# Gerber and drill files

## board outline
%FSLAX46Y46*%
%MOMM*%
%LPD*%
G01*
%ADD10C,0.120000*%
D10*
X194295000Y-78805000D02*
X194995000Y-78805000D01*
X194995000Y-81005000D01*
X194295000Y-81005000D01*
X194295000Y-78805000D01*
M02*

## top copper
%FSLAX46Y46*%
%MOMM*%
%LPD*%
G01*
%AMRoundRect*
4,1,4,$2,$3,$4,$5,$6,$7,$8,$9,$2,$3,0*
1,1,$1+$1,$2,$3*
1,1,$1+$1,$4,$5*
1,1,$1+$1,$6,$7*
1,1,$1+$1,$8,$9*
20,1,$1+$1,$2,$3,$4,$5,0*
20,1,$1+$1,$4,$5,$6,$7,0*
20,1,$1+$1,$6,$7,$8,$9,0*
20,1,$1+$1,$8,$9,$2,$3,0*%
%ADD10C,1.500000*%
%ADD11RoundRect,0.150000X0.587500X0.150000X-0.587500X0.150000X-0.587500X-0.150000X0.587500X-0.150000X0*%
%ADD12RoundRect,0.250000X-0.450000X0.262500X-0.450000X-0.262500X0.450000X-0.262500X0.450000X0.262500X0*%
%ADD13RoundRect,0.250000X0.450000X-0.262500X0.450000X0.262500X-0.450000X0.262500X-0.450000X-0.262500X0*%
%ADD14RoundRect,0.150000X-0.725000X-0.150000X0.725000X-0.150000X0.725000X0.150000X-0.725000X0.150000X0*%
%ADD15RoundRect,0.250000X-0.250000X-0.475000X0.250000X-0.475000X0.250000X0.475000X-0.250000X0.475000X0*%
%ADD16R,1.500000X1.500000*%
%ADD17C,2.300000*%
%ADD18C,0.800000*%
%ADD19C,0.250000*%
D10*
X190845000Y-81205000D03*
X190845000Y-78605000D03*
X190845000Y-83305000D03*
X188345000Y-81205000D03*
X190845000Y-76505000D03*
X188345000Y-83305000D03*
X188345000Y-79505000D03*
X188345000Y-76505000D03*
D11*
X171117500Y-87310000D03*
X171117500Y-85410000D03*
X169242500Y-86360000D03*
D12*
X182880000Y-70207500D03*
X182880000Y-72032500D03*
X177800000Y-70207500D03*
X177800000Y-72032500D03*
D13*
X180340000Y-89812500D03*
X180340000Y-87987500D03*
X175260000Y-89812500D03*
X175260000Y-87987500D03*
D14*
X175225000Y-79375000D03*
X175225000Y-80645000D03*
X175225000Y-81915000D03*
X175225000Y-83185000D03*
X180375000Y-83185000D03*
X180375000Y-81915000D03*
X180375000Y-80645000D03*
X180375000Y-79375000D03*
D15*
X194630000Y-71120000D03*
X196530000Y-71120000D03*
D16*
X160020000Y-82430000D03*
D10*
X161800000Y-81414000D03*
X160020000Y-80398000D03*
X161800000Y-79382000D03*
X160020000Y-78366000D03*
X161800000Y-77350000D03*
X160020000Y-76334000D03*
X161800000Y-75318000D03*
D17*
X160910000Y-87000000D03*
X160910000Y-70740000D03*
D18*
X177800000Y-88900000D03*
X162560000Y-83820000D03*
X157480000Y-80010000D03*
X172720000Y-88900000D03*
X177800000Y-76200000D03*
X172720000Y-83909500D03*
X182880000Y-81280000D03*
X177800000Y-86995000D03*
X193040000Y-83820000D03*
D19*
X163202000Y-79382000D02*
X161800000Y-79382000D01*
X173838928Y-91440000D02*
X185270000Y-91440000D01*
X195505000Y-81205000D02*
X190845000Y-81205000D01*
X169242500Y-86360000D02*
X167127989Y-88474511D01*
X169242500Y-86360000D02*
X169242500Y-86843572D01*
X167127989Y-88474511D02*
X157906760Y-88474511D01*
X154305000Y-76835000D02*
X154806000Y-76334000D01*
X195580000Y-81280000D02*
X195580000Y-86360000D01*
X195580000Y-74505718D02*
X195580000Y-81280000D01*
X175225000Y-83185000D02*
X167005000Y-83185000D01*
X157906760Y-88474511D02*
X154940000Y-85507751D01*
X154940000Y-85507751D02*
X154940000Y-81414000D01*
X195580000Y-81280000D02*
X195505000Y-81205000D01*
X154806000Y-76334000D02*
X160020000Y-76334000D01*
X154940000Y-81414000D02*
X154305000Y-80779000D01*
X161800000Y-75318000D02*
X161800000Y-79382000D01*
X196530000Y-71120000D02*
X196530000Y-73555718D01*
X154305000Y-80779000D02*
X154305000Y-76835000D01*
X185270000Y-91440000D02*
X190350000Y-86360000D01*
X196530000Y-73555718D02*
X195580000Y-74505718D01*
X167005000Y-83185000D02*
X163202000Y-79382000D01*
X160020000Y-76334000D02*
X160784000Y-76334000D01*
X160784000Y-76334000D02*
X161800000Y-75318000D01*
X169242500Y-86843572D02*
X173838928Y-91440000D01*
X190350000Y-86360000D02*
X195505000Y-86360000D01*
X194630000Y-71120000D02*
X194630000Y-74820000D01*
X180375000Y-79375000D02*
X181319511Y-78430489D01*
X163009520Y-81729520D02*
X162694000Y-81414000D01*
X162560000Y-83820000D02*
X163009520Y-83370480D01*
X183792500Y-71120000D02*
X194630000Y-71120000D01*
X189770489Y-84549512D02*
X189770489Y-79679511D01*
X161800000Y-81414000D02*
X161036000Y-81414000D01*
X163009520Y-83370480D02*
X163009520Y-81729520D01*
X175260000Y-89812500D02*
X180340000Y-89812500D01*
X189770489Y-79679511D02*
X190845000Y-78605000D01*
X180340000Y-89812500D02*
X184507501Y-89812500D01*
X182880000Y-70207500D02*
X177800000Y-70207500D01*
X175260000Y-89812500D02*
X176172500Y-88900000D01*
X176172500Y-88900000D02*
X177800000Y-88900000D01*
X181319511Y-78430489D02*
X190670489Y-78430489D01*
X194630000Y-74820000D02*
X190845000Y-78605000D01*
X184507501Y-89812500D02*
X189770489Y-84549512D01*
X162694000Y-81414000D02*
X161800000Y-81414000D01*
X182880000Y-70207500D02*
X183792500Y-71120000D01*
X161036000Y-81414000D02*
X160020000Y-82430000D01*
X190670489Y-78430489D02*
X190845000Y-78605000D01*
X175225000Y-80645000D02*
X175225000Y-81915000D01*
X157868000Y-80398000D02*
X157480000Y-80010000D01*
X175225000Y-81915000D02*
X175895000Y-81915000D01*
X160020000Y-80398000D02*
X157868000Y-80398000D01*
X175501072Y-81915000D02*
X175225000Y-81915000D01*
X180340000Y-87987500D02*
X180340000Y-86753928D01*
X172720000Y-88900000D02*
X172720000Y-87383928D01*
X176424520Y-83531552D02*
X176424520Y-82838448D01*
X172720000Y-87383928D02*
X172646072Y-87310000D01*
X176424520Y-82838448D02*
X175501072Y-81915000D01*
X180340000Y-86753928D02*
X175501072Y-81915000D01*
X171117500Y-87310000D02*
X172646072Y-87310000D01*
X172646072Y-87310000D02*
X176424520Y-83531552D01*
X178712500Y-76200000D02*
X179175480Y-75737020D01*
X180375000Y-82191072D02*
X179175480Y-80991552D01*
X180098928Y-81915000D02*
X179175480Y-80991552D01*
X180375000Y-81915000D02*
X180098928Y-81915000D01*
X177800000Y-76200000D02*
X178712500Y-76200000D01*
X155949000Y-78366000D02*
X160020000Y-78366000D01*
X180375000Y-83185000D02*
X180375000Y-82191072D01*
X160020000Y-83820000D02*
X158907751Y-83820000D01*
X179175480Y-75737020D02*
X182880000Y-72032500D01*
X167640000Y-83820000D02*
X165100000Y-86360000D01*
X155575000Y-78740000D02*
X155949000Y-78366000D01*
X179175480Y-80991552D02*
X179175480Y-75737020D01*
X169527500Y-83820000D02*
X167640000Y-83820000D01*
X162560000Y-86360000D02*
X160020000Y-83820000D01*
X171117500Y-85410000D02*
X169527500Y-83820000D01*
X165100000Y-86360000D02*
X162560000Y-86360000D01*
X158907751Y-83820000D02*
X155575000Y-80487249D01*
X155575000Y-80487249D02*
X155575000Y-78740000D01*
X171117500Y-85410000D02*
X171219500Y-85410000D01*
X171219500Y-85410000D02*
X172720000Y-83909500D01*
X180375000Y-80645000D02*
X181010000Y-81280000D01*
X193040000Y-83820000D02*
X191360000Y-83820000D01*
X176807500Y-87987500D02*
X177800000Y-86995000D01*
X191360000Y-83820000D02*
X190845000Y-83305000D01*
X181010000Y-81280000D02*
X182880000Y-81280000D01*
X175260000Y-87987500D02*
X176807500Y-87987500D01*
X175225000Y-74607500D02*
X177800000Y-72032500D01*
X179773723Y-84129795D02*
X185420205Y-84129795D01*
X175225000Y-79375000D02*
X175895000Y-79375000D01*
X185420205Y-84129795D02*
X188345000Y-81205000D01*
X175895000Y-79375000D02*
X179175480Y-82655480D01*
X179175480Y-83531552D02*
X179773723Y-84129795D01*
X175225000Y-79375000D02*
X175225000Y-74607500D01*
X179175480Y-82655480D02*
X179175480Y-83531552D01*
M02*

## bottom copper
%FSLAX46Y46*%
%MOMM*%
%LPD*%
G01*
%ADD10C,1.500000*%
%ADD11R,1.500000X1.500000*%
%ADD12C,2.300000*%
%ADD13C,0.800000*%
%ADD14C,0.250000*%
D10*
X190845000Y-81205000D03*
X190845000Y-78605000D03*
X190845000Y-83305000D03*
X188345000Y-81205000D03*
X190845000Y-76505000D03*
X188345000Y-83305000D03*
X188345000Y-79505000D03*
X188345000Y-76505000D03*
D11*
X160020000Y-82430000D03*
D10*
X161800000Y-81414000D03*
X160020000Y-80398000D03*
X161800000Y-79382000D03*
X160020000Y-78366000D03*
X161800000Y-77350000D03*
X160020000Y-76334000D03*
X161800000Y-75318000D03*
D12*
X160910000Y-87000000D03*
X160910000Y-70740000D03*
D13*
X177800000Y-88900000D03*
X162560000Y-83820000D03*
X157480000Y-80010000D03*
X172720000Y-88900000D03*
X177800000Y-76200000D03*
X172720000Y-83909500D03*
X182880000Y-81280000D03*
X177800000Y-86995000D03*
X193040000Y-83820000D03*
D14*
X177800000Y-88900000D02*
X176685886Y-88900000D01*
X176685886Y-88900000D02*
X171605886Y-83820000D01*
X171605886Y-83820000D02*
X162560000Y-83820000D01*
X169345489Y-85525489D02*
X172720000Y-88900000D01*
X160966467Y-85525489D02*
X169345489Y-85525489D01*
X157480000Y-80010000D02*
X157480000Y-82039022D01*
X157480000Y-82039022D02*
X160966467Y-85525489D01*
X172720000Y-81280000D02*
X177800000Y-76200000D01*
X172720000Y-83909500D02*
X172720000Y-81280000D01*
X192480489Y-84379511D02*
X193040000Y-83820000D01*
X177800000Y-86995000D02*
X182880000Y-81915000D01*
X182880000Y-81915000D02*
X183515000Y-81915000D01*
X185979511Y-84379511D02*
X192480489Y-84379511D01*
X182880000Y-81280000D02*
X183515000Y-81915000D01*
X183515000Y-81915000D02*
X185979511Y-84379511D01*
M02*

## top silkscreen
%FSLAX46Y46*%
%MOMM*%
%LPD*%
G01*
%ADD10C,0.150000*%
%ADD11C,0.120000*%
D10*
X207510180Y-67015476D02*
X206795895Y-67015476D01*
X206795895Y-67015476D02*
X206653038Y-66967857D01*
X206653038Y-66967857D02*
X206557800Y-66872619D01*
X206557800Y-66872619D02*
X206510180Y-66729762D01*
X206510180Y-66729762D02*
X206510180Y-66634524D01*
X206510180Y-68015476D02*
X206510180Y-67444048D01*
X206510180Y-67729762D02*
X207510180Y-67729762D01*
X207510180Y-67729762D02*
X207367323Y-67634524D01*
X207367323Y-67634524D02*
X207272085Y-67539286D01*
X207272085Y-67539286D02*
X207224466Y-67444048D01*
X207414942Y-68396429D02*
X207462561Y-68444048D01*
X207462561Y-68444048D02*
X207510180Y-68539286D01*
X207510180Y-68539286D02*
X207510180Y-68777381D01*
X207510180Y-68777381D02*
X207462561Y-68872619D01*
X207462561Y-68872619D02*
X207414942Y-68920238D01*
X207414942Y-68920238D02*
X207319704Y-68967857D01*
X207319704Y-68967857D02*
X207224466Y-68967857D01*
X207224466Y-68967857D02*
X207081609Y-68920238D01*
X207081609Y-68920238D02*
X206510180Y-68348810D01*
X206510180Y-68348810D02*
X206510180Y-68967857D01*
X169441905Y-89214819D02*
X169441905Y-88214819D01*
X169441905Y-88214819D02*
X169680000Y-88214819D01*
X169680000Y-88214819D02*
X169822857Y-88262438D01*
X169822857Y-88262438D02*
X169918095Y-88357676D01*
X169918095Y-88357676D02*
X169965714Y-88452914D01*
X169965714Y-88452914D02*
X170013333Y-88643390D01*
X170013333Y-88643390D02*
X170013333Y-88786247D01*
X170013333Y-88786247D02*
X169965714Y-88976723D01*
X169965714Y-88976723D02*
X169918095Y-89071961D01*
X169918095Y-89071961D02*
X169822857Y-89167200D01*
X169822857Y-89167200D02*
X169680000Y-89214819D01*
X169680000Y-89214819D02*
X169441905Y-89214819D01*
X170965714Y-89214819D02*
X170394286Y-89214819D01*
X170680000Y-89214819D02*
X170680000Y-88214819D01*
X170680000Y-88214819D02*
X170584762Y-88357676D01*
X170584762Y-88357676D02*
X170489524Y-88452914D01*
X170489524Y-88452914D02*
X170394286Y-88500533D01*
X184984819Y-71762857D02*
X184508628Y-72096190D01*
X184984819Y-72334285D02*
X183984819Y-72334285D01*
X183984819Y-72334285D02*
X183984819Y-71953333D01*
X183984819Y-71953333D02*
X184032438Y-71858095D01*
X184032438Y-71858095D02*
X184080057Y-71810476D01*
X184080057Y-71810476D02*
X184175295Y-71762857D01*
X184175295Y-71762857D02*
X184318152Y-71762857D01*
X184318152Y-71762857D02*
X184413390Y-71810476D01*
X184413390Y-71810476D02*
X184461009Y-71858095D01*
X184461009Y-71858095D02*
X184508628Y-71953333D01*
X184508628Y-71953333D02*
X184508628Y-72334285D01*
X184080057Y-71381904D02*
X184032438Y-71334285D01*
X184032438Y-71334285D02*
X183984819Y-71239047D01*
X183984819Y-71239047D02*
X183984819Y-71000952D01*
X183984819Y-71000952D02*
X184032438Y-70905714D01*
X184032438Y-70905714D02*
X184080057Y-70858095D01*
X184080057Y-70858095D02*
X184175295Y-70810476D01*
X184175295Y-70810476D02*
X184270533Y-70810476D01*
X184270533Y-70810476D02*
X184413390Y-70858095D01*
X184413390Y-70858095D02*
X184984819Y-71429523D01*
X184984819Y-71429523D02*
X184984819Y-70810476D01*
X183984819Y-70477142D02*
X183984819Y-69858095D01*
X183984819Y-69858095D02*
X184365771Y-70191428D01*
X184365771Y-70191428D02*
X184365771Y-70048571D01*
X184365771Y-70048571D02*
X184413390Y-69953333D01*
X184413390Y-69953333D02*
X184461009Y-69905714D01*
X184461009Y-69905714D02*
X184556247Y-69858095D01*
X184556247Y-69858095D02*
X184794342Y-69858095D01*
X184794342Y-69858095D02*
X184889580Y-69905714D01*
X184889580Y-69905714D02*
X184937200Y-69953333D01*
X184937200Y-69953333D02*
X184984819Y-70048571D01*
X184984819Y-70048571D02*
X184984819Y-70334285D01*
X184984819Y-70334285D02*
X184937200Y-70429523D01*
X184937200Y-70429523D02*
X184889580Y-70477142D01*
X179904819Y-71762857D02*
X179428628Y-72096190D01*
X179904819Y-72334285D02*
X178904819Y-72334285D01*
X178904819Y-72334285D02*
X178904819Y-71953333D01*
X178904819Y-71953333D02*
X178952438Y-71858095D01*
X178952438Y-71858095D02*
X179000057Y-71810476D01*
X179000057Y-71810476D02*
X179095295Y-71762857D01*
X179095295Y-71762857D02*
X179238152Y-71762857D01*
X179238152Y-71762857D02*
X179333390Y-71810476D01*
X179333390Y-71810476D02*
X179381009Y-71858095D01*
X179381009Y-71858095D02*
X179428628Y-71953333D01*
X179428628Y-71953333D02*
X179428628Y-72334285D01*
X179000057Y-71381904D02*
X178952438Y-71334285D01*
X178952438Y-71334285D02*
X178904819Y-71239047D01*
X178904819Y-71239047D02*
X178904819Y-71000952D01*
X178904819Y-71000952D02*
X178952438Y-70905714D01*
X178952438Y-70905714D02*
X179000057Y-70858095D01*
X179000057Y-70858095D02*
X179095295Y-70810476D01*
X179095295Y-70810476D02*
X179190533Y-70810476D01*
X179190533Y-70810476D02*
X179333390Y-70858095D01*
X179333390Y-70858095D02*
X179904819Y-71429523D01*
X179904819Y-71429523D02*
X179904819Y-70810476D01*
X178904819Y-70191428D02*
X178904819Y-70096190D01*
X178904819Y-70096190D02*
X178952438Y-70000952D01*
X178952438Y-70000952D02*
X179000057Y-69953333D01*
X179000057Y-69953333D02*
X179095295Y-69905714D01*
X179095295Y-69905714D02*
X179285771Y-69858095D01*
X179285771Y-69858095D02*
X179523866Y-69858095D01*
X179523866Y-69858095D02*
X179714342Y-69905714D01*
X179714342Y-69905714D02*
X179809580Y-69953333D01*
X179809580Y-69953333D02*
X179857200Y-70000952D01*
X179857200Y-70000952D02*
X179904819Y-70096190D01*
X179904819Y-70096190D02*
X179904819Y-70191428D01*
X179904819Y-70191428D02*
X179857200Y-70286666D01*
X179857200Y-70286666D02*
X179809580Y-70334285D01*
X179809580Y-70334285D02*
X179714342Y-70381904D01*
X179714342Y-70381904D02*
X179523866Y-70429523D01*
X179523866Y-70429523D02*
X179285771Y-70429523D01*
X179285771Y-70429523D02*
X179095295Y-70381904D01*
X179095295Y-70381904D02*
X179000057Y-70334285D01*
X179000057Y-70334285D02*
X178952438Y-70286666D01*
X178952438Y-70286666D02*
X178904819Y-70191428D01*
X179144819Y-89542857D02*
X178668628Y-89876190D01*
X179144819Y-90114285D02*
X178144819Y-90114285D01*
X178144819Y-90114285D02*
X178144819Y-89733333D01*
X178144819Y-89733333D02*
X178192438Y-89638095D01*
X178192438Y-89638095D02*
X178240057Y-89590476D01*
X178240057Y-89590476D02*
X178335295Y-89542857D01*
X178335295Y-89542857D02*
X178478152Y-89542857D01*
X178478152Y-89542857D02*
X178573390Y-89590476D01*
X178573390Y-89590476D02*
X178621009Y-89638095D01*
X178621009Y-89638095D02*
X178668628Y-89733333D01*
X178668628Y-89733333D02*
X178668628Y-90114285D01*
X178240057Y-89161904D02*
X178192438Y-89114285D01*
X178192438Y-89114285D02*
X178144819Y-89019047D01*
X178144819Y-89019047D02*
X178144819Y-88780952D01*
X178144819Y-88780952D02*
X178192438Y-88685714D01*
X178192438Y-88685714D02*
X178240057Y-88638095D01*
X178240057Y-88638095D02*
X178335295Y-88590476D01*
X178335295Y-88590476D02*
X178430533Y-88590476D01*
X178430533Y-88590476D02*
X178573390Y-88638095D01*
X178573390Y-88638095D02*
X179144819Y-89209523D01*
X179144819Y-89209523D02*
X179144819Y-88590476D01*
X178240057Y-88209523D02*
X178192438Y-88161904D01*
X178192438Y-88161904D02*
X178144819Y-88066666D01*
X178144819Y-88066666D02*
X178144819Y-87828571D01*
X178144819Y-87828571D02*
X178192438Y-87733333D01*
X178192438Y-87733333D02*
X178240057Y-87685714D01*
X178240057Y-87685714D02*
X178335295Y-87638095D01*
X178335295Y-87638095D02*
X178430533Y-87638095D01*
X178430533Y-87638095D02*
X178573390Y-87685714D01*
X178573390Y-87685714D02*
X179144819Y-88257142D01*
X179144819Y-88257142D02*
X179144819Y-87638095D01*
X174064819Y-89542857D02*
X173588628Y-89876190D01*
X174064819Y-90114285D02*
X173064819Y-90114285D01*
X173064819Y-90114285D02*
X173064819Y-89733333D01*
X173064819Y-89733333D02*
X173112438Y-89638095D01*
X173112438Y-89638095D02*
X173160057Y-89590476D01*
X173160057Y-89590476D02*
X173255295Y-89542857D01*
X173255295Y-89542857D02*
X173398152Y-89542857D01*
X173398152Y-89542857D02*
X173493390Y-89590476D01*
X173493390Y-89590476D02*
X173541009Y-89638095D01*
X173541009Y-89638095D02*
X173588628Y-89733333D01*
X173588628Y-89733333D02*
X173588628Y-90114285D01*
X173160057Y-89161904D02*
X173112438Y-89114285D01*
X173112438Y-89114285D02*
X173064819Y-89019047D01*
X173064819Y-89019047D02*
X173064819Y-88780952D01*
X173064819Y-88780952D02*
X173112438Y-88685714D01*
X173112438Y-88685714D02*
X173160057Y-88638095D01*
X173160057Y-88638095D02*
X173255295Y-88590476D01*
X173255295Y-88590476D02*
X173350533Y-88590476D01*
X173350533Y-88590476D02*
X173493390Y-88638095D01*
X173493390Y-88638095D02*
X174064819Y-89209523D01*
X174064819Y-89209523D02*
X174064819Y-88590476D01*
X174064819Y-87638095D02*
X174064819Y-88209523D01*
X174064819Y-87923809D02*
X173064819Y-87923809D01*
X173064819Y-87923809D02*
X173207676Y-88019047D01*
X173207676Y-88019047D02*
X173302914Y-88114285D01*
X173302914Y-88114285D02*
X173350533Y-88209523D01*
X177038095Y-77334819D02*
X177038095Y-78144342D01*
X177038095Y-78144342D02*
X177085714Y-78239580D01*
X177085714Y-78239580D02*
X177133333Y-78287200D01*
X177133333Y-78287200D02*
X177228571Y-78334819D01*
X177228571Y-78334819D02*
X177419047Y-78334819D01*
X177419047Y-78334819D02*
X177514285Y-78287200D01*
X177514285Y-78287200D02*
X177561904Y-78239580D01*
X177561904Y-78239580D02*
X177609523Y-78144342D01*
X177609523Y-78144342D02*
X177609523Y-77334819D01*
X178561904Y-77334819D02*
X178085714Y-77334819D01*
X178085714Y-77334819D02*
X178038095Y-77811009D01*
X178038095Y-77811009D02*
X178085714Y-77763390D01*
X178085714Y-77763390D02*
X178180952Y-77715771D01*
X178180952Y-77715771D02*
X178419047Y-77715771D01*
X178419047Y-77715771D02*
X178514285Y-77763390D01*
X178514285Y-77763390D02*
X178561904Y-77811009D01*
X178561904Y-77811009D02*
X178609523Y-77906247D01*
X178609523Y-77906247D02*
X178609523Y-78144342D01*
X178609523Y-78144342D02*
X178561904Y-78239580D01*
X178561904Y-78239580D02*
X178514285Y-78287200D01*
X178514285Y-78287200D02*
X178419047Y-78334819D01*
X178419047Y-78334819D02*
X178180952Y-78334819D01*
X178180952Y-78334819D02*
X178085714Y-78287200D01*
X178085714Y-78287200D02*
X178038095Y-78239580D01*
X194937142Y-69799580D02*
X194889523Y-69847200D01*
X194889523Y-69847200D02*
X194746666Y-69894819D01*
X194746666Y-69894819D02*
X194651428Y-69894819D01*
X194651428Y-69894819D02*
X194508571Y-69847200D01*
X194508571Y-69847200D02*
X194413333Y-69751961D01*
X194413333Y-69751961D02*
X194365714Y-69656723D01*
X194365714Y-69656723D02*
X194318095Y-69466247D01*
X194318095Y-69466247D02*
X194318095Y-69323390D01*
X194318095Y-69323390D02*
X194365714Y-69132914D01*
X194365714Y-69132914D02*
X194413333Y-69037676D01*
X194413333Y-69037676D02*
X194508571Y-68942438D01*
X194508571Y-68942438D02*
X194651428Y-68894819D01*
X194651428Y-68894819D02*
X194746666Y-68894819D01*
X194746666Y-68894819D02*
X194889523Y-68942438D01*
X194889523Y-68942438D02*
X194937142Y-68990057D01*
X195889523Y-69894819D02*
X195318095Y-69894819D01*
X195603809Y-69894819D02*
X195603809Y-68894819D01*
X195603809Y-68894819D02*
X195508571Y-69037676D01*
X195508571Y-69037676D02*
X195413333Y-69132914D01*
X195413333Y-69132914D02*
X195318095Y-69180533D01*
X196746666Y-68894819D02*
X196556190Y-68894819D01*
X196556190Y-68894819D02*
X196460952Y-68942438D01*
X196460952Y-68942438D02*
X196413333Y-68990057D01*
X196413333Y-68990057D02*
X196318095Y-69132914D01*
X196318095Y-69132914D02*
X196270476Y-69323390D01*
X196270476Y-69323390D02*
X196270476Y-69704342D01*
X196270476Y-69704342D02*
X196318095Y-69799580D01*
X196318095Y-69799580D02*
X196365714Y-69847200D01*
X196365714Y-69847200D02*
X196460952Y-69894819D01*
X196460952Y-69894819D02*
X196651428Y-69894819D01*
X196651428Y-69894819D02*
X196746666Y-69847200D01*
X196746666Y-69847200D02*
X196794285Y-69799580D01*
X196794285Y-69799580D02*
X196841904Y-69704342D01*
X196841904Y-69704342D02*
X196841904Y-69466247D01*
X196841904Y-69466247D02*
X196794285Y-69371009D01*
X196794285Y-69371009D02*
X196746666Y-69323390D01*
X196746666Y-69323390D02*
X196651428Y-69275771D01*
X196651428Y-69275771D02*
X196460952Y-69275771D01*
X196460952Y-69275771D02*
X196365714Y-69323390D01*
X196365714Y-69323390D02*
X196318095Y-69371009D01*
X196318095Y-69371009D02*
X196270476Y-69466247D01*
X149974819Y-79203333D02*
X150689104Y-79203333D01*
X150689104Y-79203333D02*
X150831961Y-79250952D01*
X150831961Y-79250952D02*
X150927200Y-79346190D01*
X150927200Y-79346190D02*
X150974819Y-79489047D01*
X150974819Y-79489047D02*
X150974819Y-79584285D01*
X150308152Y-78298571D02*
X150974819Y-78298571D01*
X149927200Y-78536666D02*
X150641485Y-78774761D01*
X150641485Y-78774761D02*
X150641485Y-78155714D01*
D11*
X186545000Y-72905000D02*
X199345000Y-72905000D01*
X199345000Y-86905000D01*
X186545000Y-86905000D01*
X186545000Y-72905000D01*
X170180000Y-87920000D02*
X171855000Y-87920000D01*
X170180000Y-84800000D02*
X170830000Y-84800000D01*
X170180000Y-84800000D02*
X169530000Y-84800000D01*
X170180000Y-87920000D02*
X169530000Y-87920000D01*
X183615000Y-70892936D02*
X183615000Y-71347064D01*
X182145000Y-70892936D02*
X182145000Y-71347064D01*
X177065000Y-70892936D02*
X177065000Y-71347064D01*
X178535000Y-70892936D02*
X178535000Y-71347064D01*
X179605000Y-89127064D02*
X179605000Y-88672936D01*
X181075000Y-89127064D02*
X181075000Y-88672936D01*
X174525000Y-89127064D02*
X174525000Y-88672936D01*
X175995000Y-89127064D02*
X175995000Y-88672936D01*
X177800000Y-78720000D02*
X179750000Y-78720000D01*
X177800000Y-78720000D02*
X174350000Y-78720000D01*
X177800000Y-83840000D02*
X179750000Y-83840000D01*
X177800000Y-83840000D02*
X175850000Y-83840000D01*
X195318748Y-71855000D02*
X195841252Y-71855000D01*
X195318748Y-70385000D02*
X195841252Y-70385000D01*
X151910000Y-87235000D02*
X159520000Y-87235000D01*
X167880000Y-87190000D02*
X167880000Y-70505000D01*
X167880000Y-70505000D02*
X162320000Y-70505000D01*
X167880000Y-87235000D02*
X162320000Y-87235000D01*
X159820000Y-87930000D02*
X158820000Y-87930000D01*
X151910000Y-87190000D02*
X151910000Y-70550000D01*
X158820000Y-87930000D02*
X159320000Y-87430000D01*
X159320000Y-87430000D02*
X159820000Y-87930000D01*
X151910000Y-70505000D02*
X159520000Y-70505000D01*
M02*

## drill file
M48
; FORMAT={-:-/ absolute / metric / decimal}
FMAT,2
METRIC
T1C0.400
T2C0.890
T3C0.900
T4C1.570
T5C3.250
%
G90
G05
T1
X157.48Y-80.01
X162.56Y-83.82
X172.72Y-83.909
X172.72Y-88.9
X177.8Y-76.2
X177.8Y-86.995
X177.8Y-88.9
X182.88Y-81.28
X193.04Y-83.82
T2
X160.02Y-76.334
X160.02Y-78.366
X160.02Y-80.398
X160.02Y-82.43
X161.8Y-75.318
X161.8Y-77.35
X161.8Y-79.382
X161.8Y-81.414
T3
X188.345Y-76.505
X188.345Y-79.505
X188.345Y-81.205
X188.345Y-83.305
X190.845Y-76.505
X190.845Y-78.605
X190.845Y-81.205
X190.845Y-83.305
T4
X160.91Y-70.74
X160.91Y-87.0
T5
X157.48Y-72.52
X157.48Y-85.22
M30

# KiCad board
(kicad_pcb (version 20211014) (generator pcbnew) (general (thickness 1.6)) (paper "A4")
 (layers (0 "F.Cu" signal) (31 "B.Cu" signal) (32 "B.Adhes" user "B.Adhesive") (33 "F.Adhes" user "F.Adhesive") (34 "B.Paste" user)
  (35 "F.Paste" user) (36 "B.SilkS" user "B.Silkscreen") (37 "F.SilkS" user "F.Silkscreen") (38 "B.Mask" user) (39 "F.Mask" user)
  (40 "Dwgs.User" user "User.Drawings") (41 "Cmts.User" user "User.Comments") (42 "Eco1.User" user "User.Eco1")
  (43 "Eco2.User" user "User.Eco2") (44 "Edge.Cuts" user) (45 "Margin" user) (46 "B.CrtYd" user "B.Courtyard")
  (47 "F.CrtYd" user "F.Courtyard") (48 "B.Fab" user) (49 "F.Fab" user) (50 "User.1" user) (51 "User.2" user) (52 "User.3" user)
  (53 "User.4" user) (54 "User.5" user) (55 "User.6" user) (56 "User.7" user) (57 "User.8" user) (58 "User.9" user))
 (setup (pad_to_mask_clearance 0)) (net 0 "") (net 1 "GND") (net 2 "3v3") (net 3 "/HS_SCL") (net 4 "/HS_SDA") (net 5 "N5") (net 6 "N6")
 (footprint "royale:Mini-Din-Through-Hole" (layer "F.Cu") (at 199.345 72.905 -90)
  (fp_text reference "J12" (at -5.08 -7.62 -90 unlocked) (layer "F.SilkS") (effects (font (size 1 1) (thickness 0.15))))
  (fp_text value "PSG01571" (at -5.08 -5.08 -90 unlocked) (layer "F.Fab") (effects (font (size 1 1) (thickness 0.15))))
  (fp_rect (start 0 0) (end 14 12.8) (layer "F.SilkS") (width 0.12) (fill none))
  (fp_rect (start 5.9 4.35) (end 8.1 5.05) (layer "Edge.Cuts") (width 0.12) (fill none))
  (pad "1" thru_hole circle (at 8.3 8.5 270) (size 1.5 1.5) (drill 0.9) (layers *.Cu *.Mask) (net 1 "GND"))
  (pad "2" thru_hole circle (at 5.7 8.5 270) (size 1.5 1.5) (drill 0.9) (layers *.Cu *.Mask) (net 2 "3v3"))
  (pad "3" thru_hole circle (at 10.4 8.5 270) (size 1.5 1.5) (drill 0.9) (layers *.Cu *.Mask) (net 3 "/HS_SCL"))
  (pad "4" thru_hole circle (at 8.3 11 270) (size 1.5 1.5) (drill 0.9) (layers *.Cu *.Mask) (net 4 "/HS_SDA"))
  (pad "5" thru_hole circle (at 3.6 8.5 270) (size 1.5 1.5) (drill 0.9) (layers *.Cu *.Mask))
  (pad "6" thru_hole circle (at 10.4 11 270) (size 1.5 1.5) (drill 0.9) (layers *.Cu *.Mask))
  (pad "7" thru_hole circle (at 6.6 11 270) (size 1.5 1.5) (drill 0.9) (layers *.Cu *.Mask))
  (pad "8" thru_hole circle (at 3.6 11 270) (size 1.5 1.5) (drill 0.9) (layers *.Cu *.Mask)))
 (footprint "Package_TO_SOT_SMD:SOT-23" (layer "F.Cu") (at 170.18 86.36 180)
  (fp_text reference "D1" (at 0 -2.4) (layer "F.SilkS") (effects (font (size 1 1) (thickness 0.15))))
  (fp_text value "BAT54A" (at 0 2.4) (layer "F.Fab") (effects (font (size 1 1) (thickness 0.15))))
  (fp_line (start 0 -1.56) (end -1.675 -1.56) (layer "F.SilkS") (width 0.12))
  (fp_line (start 0 1.56) (end -0.65 1.56) (layer "F.SilkS") (width 0.12))
  (fp_line (start 0 1.56) (end 0.65 1.56) (layer "F.SilkS") (width 0.12))
  (fp_line (start 0 -1.56) (end 0.65 -1.56) (layer "F.SilkS") (width 0.12))
  (pad "1" smd roundrect (at -0.9375 -0.95 180) (size 1.475 0.6) (layers "F.Cu" "F.Paste" "F.Mask") (roundrect_rratio 0.25) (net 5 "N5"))
  (pad "2" smd roundrect (at -0.9375 0.95 180) (size 1.475 0.6) (layers "F.Cu" "F.Paste" "F.Mask") (roundrect_rratio 0.25) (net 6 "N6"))
  (pad "3" smd roundrect (at 0.9375 0 180) (size 1.475 0.6) (layers "F.Cu" "F.Paste" "F.Mask") (roundrect_rratio 0.25) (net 1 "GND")))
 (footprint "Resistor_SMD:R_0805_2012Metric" (layer "F.Cu") (at 182.88 71.12 -90)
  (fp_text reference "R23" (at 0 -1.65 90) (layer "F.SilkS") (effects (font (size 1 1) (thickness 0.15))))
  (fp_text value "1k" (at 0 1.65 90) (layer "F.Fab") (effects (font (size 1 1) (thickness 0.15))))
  (fp_line (start -0.227064 -0.735) (end 0.227064 -0.735) (layer "F.SilkS") (width 0.12))
  (fp_line (start -0.227064 0.735) (end 0.227064 0.735) (layer "F.SilkS") (width 0.12))
  (pad "1" smd roundrect (at -0.9125 0 270) (size 1.025 1.4) (layers "F.Cu" "F.Paste" "F.Mask") (roundrect_rratio 0.243902) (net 2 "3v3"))
  (pad "2" smd roundrect (at 0.9125 0 270) (size 1.025 1.4) (layers "F.Cu" "F.Paste" "F.Mask") (roundrect_rratio 0.243902) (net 6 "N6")))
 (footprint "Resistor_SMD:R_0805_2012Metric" (layer "F.Cu") (at 177.8 71.12 -90)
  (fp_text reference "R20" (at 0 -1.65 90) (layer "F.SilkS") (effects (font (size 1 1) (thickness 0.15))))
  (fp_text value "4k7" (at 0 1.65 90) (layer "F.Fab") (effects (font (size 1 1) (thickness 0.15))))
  (fp_line (start -0.227064 0.735) (end 0.227064 0.735) (layer "F.SilkS") (width 0.12))
  (fp_line (start -0.227064 -0.735) (end 0.227064 -0.735) (layer "F.SilkS") (width 0.12))
  (pad "1" smd roundrect (at -0.9125 0 270) (size 1.025 1.4) (layers "F.Cu" "F.Paste" "F.Mask") (roundrect_rratio 0.243902) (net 2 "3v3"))
  (pad "2" smd roundrect (at 0.9125 0 270) (size 1.025 1.4) (layers "F.Cu" "F.Paste" "F.Mask") (roundrect_rratio 0.243902) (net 4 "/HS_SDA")))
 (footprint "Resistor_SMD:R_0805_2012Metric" (layer "F.Cu") (at 180.34 88.9 90)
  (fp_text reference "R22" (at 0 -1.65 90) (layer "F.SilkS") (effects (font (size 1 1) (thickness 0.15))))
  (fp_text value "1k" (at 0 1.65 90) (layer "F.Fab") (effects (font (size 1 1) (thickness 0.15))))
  (fp_line (start -0.227064 -0.735) (end 0.227064 -0.735) (layer "F.SilkS") (width 0.12))
  (fp_line (start -0.227064 0.735) (end 0.227064 0.735) (layer "F.SilkS") (width 0.12))
  (pad "1" smd roundrect (at -0.9125 0 90) (size 1.025 1.4) (layers "F.Cu" "F.Paste" "F.Mask") (roundrect_rratio 0.243902) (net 2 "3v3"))
  (pad "2" smd roundrect (at 0.9125 0 90) (size 1.025 1.4) (layers "F.Cu" "F.Paste" "F.Mask") (roundrect_rratio 0.243902) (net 5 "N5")))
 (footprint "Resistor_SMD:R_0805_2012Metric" (layer "F.Cu") (at 175.26 88.9 90)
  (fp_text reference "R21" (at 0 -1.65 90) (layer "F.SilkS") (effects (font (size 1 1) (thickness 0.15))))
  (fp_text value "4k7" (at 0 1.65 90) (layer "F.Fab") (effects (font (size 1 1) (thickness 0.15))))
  (fp_line (start -0.227064 -0.735) (end 0.227064 -0.735) (layer "F.SilkS") (width 0.12))
  (fp_line (start -0.227064 0.735) (end 0.227064 0.735) (layer "F.SilkS") (width 0.12))
  (pad "1" smd roundrect (at -0.9125 0 90) (size 1.025 1.4) (layers "F.Cu" "F.Paste" "F.Mask") (roundrect_rratio 0.243902) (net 2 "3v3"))
  (pad "2" smd roundrect (at 0.9125 0 90) (size 1.025 1.4) (layers "F.Cu" "F.Paste" "F.Mask") (roundrect_rratio 0.243902) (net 3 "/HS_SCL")))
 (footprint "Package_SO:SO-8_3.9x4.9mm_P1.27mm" (layer "F.Cu") (at 177.8 81.28)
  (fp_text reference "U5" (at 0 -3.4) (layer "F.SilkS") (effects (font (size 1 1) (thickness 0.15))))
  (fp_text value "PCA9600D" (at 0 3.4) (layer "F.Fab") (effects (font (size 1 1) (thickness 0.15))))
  (fp_line (start 0 -2.56) (end 1.95 -2.56) (layer "F.SilkS") (width 0.12))
  (fp_line (start 0 -2.56) (end -3.45 -2.56) (layer "F.SilkS") (width 0.12))
  (fp_line (start 0 2.56) (end 1.95 2.56) (layer "F.SilkS") (width 0.12))
  (fp_line (start 0 2.56) (end -1.95 2.56) (layer "F.SilkS") (width 0.12))
  (pad "1" smd roundrect (at -2.575 -1.905) (size 1.75 0.6) (layers "F.Cu" "F.Paste" "F.Mask") (roundrect_rratio 0.25) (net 4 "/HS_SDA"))
  (pad "2" smd roundrect (at -2.575 -0.635) (size 1.75 0.6) (layers "F.Cu" "F.Paste" "F.Mask") (roundrect_rratio 0.25) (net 5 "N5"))
  (pad "3" smd roundrect (at -2.575 0.635) (size 1.75 0.6) (layers "F.Cu" "F.Paste" "F.Mask") (roundrect_rratio 0.25) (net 5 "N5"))
  (pad "4" smd roundrect (at -2.575 1.905) (size 1.75 0.6) (layers "F.Cu" "F.Paste" "F.Mask") (roundrect_rratio 0.25) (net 1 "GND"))
  (pad "5" smd roundrect (at 2.575 1.905) (size 1.75 0.6) (layers "F.Cu" "F.Paste" "F.Mask") (roundrect_rratio 0.25) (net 6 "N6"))
  (pad "6" smd roundrect (at 2.575 0.635) (size 1.75 0.6) (layers "F.Cu" "F.Paste" "F.Mask") (roundrect_rratio 0.25) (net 6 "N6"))
  (pad "7" smd roundrect (at 2.575 -0.635) (size 1.75 0.6) (layers "F.Cu" "F.Paste" "F.Mask") (roundrect_rratio 0.25) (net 3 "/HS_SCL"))
  (pad "8" smd roundrect (at 2.575 -1.905) (size 1.75 0.6) (layers "F.Cu" "F.Paste" "F.Mask") (roundrect_rratio 0.25) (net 2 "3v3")))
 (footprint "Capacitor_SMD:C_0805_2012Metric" (layer "F.Cu") (at 195.58 71.12)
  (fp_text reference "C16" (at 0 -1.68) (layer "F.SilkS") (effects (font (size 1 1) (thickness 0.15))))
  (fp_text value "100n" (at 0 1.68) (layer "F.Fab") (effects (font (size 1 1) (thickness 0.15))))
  (fp_line (start -0.261252 0.735) (end 0.261252 0.735) (layer "F.SilkS") (width 0.12))
  (fp_line (start -0.261252 -0.735) (end 0.261252 -0.735) (layer "F.SilkS") (width 0.12))
  (pad "1" smd roundrect (at -0.95 0) (size 1 1.45) (layers "F.Cu" "F.Paste" "F.Mask") (roundrect_rratio 0.25) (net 2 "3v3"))
  (pad "2" smd roundrect (at 0.95 0) (size 1 1.45) (layers "F.Cu" "F.Paste" "F.Mask") (roundrect_rratio 0.25) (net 1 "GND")))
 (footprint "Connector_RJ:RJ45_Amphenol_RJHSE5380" (layer "F.Cu") (at 160.02 82.43 90)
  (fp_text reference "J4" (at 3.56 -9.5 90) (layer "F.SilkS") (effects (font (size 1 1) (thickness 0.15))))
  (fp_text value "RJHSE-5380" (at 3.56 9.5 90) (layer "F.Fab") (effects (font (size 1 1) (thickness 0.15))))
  (fp_line (start -4.805 -8.11) (end -4.805 -0.5) (layer "F.SilkS") (width 0.12))
  (fp_line (start -4.76 7.86) (end 11.925 7.86) (layer "F.SilkS") (width 0.12))
  (fp_line (start 11.925 7.86) (end 11.925 2.3) (layer "F.SilkS") (width 0.12))
  (fp_line (start -4.805 7.86) (end -4.805 2.3) (layer "F.SilkS") (width 0.12))
  (fp_line (start -5.5 -0.2) (end -5.5 -1.2) (layer "F.SilkS") (width 0.12))
  (fp_line (start -4.76 -8.11) (end 11.88 -8.11) (layer "F.SilkS") (width 0.12))
  (fp_line (start -5.5 -1.2) (end -5 -0.7) (layer "F.SilkS") (width 0.12))
  (fp_line (start -5 -0.7) (end -5.5 -0.2) (layer "F.SilkS") (width 0.12))
  (fp_line (start 11.925 -8.11) (end 11.925 -0.5) (layer "F.SilkS") (width 0.12))
  (pad "" np_thru_hole circle (at 9.91 -2.54 90) (size 3.25 3.25) (drill 3.25) (layers *.Cu *.Mask))
  (pad "" np_thru_hole circle (at -2.79 -2.54 90) (size 3.25 3.25) (drill 3.25) (layers *.Cu *.Mask))
  (pad "1" thru_hole rect (at 0 0 90) (size 1.5 1.5) (drill 0.89) (layers *.Cu *.Mask) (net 2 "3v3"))
  (pad "2" thru_hole circle (at 1.016 1.78 90) (size 1.5 1.5) (drill 0.89) (layers *.Cu *.Mask) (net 2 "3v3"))
  (pad "3" thru_hole circle (at 2.032 0 90) (size 1.5 1.5) (drill 0.89) (layers *.Cu *.Mask) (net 5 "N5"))
  (pad "4" thru_hole circle (at 3.048 1.78 90) (size 1.5 1.5) (drill 0.89) (layers *.Cu *.Mask) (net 1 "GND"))
  (pad "5" thru_hole circle (at 4.064 0 90) (size 1.5 1.5) (drill 0.89) (layers *.Cu *.Mask) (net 6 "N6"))
  (pad "6" thru_hole circle (at 5.08 1.78 90) (size 1.5 1.5) (drill 0.89) (layers *.Cu *.Mask) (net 1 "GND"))
  (pad "7" thru_hole circle (at 6.096 0 90) (size 1.5 1.5) (drill 0.89) (layers *.Cu *.Mask) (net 1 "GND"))
  (pad "8" thru_hole circle (at 7.112 1.78 90) (size 1.5 1.5) (drill 0.89) (layers *.Cu *.Mask) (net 1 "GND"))
  (pad "SH" thru_hole circle (at -4.57 0.89 90) (size 2.3 2.3) (drill 1.57) (layers *.Cu *.Mask))
  (pad "SH" thru_hole circle (at 11.69 0.89 90) (size 2.3 2.3) (drill 1.57) (layers *.Cu *.Mask)))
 (segment (start 163.202 79.382) (end 161.8 79.382) (width 0.25) (layer "F.Cu") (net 1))
 (segment (start 173.838928 91.44) (end 185.27 91.44) (width 0.25) (layer "F.Cu") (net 1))
 (segment (start 195.505 81.205) (end 190.845 81.205) (width 0.25) (layer "F.Cu") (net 1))
 (segment (start 169.2425 86.36) (end 167.127989 88.474511) (width 0.25) (layer "F.Cu") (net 1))
 (segment (start 169.2425 86.36) (end 169.2425 86.843572) (width 0.25) (layer "F.Cu") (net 1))
 (segment (start 167.127989 88.474511) (end 157.90676 88.474511) (width 0.25) (layer "F.Cu") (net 1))
 (segment (start 154.305 76.835) (end 154.806 76.334) (width 0.25) (layer "F.Cu") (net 1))
 (segment (start 195.58 81.28) (end 195.58 86.36) (width 0.25) (layer "F.Cu") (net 1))
 (segment (start 195.58 74.505718) (end 195.58 81.28) (width 0.25) (layer "F.Cu") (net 1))
 (segment (start 175.225 83.185) (end 167.005 83.185) (width 0.25) (layer "F.Cu") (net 1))
 (segment (start 157.90676 88.474511) (end 154.94 85.507751) (width 0.25) (layer "F.Cu") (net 1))
 (segment (start 154.94 85.507751) (end 154.94 81.414) (width 0.25) (layer "F.Cu") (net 1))
 (segment (start 195.58 81.28) (end 195.505 81.205) (width 0.25) (layer "F.Cu") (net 1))
 (segment (start 154.806 76.334) (end 160.02 76.334) (width 0.25) (layer "F.Cu") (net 1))
 (segment (start 154.94 81.414) (end 154.305 80.779) (width 0.25) (layer "F.Cu") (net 1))
 (segment (start 161.8 75.318) (end 161.8 79.382) (width 0.25) (layer "F.Cu") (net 1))
 (segment (start 196.53 71.12) (end 196.53 73.555718) (width 0.25) (layer "F.Cu") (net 1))
 (segment (start 154.305 80.779) (end 154.305 76.835) (width 0.25) (layer "F.Cu") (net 1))
 (segment (start 185.27 91.44) (end 190.35 86.36) (width 0.25) (layer "F.Cu") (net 1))
 (segment (start 196.53 73.555718) (end 195.58 74.505718) (width 0.25) (layer "F.Cu") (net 1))
 (segment (start 167.005 83.185) (end 163.202 79.382) (width 0.25) (layer "F.Cu") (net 1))
 (segment (start 160.02 76.334) (end 160.784 76.334) (width 0.25) (layer "F.Cu") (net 1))
 (segment (start 160.784 76.334) (end 161.8 75.318) (width 0.25) (layer "F.Cu") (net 1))
 (segment (start 169.2425 86.843572) (end 173.838928 91.44) (width 0.25) (layer "F.Cu") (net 1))
 (segment (start 190.35 86.36) (end 195.505 86.36) (width 0.25) (layer "F.Cu") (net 1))
 (segment (start 194.63 71.12) (end 194.63 74.82) (width 0.25) (layer "F.Cu") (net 2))
 (segment (start 180.375 79.375) (end 181.319511 78.430489) (width 0.25) (layer "F.Cu") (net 2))
 (segment (start 163.00952 81.72952) (end 162.694 81.414) (width 0.25) (layer "F.Cu") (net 2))
 (segment (start 162.56 83.82) (end 163.00952 83.37048) (width 0.25) (layer "F.Cu") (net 2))
 (segment (start 183.7925 71.12) (end 194.63 71.12) (width 0.25) (layer "F.Cu") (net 2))
 (segment (start 189.770489 84.549512) (end 189.770489 79.679511) (width 0.25) (layer "F.Cu") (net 2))
 (segment (start 161.8 81.414) (end 161.036 81.414) (width 0.25) (layer "F.Cu") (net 2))
 (segment (start 163.00952 83.37048) (end 163.00952 81.72952) (width 0.25) (layer "F.Cu") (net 2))
 (segment (start 175.26 89.8125) (end 180.34 89.8125) (width 0.25) (layer "F.Cu") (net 2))
 (segment (start 189.770489 79.679511) (end 190.845 78.605) (width 0.25) (layer "F.Cu") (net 2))
 (segment (start 180.34 89.8125) (end 184.507501 89.8125) (width 0.25) (layer "F.Cu") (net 2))
 (segment (start 182.88 70.2075) (end 177.8 70.2075) (width 0.25) (layer "F.Cu") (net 2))
 (segment (start 175.26 89.8125) (end 176.1725 88.9) (width 0.25) (layer "F.Cu") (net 2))
 (segment (start 176.1725 88.9) (end 177.8 88.9) (width 0.25) (layer "F.Cu") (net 2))
 (segment (start 181.319511 78.430489) (end 190.670489 78.430489) (width 0.25) (layer "F.Cu") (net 2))
 (segment (start 194.63 74.82) (end 190.845 78.605) (width 0.25) (layer "F.Cu") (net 2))
 (segment (start 184.507501 89.8125) (end 189.770489 84.549512) (width 0.25) (layer "F.Cu") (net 2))
 (segment (start 162.694 81.414) (end 161.8 81.414) (width 0.25) (layer "F.Cu") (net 2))
 (segment (start 182.88 70.2075) (end 183.7925 71.12) (width 0.25) (layer "F.Cu") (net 2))
 (segment (start 161.036 81.414) (end 160.02 82.43) (width 0.25) (layer "F.Cu") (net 2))
 (segment (start 190.670489 78.430489) (end 190.845 78.605) (width 0.25) (layer "F.Cu") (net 2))
 (via (at 177.8 88.9) (size 0.8) (drill 0.4) (layers "F.Cu" "B.Cu") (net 2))
 (via (at 162.56 83.82) (size 0.8) (drill 0.4) (layers "F.Cu" "B.Cu") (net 2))
 (segment (start 177.8 88.9) (end 176.685886 88.9) (width 0.25) (layer "B.Cu") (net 2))
 (segment (start 176.685886 88.9) (end 171.605886 83.82) (width 0.25) (layer "B.Cu") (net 2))
 (segment (start 171.605886 83.82) (end 162.56 83.82) (width 0.25) (layer "B.Cu") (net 2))
 (segment (start 175.225 80.645) (end 175.225 81.915) (width 0.25) (layer "F.Cu") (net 5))
 (segment (start 157.868 80.398) (end 157.48 80.01) (width 0.25) (layer "F.Cu") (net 5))
 (segment (start 175.225 81.915) (end 175.895 81.915) (width 0.25) (layer "F.Cu") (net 5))
 (segment (start 160.02 80.398) (end 157.868 80.398) (width 0.25) (layer "F.Cu") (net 5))
 (segment (start 175.501072 81.915) (end 175.225 81.915) (width 0.25) (layer "F.Cu") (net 5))
 (segment (start 180.34 87.9875) (end 180.34 86.753928) (width 0.25) (layer "F.Cu") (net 5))
 (segment (start 172.72 88.9) (end 172.72 87.383928) (width 0.25) (layer "F.Cu") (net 5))
 (segment (start 176.42452 83.531552) (end 176.42452 82.838448) (width 0.25) (layer "F.Cu") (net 5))
 (segment (start 172.72 87.383928) (end 172.646072 87.31) (width 0.25) (layer "F.Cu") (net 5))
 (segment (start 176.42452 82.838448) (end 175.501072 81.915) (width 0.25) (layer "F.Cu") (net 5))
 (segment (start 180.34 86.753928) (end 175.501072 81.915) (width 0.25) (layer "F.Cu") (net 5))
 (segment (start 171.1175 87.31) (end 172.646072 87.31) (width 0.25) (layer "F.Cu") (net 5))
 (segment (start 172.646072 87.31) (end 176.42452 83.531552) (width 0.25) (layer "F.Cu") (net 5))
 (via (at 157.48 80.01) (size 0.8) (drill 0.4) (layers "F.Cu" "B.Cu") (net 5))
 (via (at 172.72 88.9) (size 0.8) (drill 0.4) (layers "F.Cu" "B.Cu") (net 5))
 (segment (start 169.345489 85.525489) (end 172.72 88.9) (width 0.25) (layer "B.Cu") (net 5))
 (segment (start 160.966467 85.525489) (end 169.345489 85.525489) (width 0.25) (layer "B.Cu") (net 5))
 (segment (start 157.48 80.01) (end 157.48 82.039022) (width 0.25) (layer "B.Cu") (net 5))
 (segment (start 157.48 82.039022) (end 160.966467 85.525489) (width 0.25) (layer "B.Cu") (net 5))
 (segment (start 178.7125 76.2) (end 179.17548 75.73702) (width 0.25) (layer "F.Cu") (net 6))
 (segment (start 180.375 82.191072) (end 179.17548 80.991552) (width 0.25) (layer "F.Cu") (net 6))
 (segment (start 180.098928 81.915) (end 179.17548 80.991552) (width 0.25) (layer "F.Cu") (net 6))
 (segment (start 180.375 81.915) (end 180.098928 81.915) (width 0.25) (layer "F.Cu") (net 6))
 (segment (start 177.8 76.2) (end 178.7125 76.2) (width 0.25) (layer "F.Cu") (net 6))
 (segment (start 155.949 78.366) (end 160.02 78.366) (width 0.25) (layer "F.Cu") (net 6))
 (segment (start 180.375 83.185) (end 180.375 82.191072) (width 0.25) (layer "F.Cu") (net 6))
 (segment (start 160.02 83.82) (end 158.907751 83.82) (width 0.25) (layer "F.Cu") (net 6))
 (segment (start 179.17548 75.73702) (end 182.88 72.0325) (width 0.25) (layer "F.Cu") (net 6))
 (segment (start 167.64 83.82) (end 165.1 86.36) (width 0.25) (layer "F.Cu") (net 6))
 (segment (start 155.575 78.74) (end 155.949 78.366) (width 0.25) (layer "F.Cu") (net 6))
 (segment (start 179.17548 80.991552) (end 179.17548 75.73702) (width 0.25) (layer "F.Cu") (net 6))
 (segment (start 169.5275 83.82) (end 167.64 83.82) (width 0.25) (layer "F.Cu") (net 6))
 (segment (start 162.56 86.36) (end 160.02 83.82) (width 0.25) (layer "F.Cu") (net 6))
 (segment (start 171.1175 85.41) (end 169.5275 83.82) (width 0.25) (layer "F.Cu") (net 6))
 (segment (start 165.1 86.36) (end 162.56 86.36) (width 0.25) (layer "F.Cu") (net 6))
 (segment (start 158.907751 83.82) (end 155.575 80.487249) (width 0.25) (layer "F.Cu") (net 6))
 (segment (start 155.575 80.487249) (end 155.575 78.74) (width 0.25) (layer "F.Cu") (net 6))
 (segment (start 171.1175 85.41) (end 171.2195 85.41) (width 0.25) (layer "F.Cu") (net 6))
 (segment (start 171.2195 85.41) (end 172.72 83.9095) (width 0.25) (layer "F.Cu") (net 6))
 (via (at 177.8 76.2) (size 0.8) (drill 0.4) (layers "F.Cu" "B.Cu") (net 6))
 (via (at 172.72 83.9095) (size 0.8) (drill 0.4) (layers "F.Cu" "B.Cu") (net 6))
 (segment (start 172.72 81.28) (end 177.8 76.2) (width 0.25) (layer "B.Cu") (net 6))
 (segment (start 172.72 83.9095) (end 172.72 81.28) (width 0.25) (layer "B.Cu") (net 6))
 (segment (start 180.375 80.645) (end 181.01 81.28) (width 0.25) (layer "F.Cu") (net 3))
 (segment (start 193.04 83.82) (end 191.36 83.82) (width 0.25) (layer "F.Cu") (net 3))
 (segment (start 176.8075 87.9875) (end 177.8 86.995) (width 0.25) (layer "F.Cu") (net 3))
 (segment (start 191.36 83.82) (end 190.845 83.305) (width 0.25) (layer "F.Cu") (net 3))
 (segment (start 181.01 81.28) (end 182.88 81.28) (width 0.25) (layer "F.Cu") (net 3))
 (segment (start 175.26 87.9875) (end 176.8075 87.9875) (width 0.25) (layer "F.Cu") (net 3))
 (via (at 182.88 81.28) (size 0.8) (drill 0.4) (layers "F.Cu" "B.Cu") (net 3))
 (via (at 177.8 86.995) (size 0.8) (drill 0.4) (layers "F.Cu" "B.Cu") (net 3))
 (via (at 193.04 83.82) (size 0.8) (drill 0.4) (layers "F.Cu" "B.Cu") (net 3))
 (segment (start 192.480489 84.379511) (end 193.04 83.82) (width 0.25) (layer "B.Cu") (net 3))
 (segment (start 177.8 86.995) (end 182.88 81.915) (width 0.25) (layer "B.Cu") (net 3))
 (segment (start 182.88 81.915) (end 183.515 81.915) (width 0.25) (layer "B.Cu") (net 3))
 (segment (start 185.979511 84.379511) (end 192.480489 84.379511) (width 0.25) (layer "B.Cu") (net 3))
 (segment (start 182.88 81.28) (end 183.515 81.915) (width 0.25) (layer "B.Cu") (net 3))
 (segment (start 183.515 81.915) (end 185.979511 84.379511) (width 0.25) (layer "B.Cu") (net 3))
 (segment (start 175.225 74.6075) (end 177.8 72.0325) (width 0.25) (layer "F.Cu") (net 4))
 (segment (start 179.773723 84.129795) (end 185.420205 84.129795) (width 0.25) (layer "F.Cu") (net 4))
 (segment (start 175.225 79.375) (end 175.895 79.375) (width 0.25) (layer "F.Cu") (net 4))
 (segment (start 185.420205 84.129795) (end 188.345 81.205) (width 0.25) (layer "F.Cu") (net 4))
 (segment (start 175.895 79.375) (end 179.17548 82.65548) (width 0.25) (layer "F.Cu") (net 4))
 (segment (start 179.17548 83.531552) (end 179.773723 84.129795) (width 0.25) (layer "F.Cu") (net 4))
 (segment (start 175.225 79.375) (end 175.225 74.6075) (width 0.25) (layer "F.Cu") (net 4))
 (segment (start 179.17548 82.65548) (end 179.17548 83.531552) (width 0.25) (layer "F.Cu") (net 4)))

